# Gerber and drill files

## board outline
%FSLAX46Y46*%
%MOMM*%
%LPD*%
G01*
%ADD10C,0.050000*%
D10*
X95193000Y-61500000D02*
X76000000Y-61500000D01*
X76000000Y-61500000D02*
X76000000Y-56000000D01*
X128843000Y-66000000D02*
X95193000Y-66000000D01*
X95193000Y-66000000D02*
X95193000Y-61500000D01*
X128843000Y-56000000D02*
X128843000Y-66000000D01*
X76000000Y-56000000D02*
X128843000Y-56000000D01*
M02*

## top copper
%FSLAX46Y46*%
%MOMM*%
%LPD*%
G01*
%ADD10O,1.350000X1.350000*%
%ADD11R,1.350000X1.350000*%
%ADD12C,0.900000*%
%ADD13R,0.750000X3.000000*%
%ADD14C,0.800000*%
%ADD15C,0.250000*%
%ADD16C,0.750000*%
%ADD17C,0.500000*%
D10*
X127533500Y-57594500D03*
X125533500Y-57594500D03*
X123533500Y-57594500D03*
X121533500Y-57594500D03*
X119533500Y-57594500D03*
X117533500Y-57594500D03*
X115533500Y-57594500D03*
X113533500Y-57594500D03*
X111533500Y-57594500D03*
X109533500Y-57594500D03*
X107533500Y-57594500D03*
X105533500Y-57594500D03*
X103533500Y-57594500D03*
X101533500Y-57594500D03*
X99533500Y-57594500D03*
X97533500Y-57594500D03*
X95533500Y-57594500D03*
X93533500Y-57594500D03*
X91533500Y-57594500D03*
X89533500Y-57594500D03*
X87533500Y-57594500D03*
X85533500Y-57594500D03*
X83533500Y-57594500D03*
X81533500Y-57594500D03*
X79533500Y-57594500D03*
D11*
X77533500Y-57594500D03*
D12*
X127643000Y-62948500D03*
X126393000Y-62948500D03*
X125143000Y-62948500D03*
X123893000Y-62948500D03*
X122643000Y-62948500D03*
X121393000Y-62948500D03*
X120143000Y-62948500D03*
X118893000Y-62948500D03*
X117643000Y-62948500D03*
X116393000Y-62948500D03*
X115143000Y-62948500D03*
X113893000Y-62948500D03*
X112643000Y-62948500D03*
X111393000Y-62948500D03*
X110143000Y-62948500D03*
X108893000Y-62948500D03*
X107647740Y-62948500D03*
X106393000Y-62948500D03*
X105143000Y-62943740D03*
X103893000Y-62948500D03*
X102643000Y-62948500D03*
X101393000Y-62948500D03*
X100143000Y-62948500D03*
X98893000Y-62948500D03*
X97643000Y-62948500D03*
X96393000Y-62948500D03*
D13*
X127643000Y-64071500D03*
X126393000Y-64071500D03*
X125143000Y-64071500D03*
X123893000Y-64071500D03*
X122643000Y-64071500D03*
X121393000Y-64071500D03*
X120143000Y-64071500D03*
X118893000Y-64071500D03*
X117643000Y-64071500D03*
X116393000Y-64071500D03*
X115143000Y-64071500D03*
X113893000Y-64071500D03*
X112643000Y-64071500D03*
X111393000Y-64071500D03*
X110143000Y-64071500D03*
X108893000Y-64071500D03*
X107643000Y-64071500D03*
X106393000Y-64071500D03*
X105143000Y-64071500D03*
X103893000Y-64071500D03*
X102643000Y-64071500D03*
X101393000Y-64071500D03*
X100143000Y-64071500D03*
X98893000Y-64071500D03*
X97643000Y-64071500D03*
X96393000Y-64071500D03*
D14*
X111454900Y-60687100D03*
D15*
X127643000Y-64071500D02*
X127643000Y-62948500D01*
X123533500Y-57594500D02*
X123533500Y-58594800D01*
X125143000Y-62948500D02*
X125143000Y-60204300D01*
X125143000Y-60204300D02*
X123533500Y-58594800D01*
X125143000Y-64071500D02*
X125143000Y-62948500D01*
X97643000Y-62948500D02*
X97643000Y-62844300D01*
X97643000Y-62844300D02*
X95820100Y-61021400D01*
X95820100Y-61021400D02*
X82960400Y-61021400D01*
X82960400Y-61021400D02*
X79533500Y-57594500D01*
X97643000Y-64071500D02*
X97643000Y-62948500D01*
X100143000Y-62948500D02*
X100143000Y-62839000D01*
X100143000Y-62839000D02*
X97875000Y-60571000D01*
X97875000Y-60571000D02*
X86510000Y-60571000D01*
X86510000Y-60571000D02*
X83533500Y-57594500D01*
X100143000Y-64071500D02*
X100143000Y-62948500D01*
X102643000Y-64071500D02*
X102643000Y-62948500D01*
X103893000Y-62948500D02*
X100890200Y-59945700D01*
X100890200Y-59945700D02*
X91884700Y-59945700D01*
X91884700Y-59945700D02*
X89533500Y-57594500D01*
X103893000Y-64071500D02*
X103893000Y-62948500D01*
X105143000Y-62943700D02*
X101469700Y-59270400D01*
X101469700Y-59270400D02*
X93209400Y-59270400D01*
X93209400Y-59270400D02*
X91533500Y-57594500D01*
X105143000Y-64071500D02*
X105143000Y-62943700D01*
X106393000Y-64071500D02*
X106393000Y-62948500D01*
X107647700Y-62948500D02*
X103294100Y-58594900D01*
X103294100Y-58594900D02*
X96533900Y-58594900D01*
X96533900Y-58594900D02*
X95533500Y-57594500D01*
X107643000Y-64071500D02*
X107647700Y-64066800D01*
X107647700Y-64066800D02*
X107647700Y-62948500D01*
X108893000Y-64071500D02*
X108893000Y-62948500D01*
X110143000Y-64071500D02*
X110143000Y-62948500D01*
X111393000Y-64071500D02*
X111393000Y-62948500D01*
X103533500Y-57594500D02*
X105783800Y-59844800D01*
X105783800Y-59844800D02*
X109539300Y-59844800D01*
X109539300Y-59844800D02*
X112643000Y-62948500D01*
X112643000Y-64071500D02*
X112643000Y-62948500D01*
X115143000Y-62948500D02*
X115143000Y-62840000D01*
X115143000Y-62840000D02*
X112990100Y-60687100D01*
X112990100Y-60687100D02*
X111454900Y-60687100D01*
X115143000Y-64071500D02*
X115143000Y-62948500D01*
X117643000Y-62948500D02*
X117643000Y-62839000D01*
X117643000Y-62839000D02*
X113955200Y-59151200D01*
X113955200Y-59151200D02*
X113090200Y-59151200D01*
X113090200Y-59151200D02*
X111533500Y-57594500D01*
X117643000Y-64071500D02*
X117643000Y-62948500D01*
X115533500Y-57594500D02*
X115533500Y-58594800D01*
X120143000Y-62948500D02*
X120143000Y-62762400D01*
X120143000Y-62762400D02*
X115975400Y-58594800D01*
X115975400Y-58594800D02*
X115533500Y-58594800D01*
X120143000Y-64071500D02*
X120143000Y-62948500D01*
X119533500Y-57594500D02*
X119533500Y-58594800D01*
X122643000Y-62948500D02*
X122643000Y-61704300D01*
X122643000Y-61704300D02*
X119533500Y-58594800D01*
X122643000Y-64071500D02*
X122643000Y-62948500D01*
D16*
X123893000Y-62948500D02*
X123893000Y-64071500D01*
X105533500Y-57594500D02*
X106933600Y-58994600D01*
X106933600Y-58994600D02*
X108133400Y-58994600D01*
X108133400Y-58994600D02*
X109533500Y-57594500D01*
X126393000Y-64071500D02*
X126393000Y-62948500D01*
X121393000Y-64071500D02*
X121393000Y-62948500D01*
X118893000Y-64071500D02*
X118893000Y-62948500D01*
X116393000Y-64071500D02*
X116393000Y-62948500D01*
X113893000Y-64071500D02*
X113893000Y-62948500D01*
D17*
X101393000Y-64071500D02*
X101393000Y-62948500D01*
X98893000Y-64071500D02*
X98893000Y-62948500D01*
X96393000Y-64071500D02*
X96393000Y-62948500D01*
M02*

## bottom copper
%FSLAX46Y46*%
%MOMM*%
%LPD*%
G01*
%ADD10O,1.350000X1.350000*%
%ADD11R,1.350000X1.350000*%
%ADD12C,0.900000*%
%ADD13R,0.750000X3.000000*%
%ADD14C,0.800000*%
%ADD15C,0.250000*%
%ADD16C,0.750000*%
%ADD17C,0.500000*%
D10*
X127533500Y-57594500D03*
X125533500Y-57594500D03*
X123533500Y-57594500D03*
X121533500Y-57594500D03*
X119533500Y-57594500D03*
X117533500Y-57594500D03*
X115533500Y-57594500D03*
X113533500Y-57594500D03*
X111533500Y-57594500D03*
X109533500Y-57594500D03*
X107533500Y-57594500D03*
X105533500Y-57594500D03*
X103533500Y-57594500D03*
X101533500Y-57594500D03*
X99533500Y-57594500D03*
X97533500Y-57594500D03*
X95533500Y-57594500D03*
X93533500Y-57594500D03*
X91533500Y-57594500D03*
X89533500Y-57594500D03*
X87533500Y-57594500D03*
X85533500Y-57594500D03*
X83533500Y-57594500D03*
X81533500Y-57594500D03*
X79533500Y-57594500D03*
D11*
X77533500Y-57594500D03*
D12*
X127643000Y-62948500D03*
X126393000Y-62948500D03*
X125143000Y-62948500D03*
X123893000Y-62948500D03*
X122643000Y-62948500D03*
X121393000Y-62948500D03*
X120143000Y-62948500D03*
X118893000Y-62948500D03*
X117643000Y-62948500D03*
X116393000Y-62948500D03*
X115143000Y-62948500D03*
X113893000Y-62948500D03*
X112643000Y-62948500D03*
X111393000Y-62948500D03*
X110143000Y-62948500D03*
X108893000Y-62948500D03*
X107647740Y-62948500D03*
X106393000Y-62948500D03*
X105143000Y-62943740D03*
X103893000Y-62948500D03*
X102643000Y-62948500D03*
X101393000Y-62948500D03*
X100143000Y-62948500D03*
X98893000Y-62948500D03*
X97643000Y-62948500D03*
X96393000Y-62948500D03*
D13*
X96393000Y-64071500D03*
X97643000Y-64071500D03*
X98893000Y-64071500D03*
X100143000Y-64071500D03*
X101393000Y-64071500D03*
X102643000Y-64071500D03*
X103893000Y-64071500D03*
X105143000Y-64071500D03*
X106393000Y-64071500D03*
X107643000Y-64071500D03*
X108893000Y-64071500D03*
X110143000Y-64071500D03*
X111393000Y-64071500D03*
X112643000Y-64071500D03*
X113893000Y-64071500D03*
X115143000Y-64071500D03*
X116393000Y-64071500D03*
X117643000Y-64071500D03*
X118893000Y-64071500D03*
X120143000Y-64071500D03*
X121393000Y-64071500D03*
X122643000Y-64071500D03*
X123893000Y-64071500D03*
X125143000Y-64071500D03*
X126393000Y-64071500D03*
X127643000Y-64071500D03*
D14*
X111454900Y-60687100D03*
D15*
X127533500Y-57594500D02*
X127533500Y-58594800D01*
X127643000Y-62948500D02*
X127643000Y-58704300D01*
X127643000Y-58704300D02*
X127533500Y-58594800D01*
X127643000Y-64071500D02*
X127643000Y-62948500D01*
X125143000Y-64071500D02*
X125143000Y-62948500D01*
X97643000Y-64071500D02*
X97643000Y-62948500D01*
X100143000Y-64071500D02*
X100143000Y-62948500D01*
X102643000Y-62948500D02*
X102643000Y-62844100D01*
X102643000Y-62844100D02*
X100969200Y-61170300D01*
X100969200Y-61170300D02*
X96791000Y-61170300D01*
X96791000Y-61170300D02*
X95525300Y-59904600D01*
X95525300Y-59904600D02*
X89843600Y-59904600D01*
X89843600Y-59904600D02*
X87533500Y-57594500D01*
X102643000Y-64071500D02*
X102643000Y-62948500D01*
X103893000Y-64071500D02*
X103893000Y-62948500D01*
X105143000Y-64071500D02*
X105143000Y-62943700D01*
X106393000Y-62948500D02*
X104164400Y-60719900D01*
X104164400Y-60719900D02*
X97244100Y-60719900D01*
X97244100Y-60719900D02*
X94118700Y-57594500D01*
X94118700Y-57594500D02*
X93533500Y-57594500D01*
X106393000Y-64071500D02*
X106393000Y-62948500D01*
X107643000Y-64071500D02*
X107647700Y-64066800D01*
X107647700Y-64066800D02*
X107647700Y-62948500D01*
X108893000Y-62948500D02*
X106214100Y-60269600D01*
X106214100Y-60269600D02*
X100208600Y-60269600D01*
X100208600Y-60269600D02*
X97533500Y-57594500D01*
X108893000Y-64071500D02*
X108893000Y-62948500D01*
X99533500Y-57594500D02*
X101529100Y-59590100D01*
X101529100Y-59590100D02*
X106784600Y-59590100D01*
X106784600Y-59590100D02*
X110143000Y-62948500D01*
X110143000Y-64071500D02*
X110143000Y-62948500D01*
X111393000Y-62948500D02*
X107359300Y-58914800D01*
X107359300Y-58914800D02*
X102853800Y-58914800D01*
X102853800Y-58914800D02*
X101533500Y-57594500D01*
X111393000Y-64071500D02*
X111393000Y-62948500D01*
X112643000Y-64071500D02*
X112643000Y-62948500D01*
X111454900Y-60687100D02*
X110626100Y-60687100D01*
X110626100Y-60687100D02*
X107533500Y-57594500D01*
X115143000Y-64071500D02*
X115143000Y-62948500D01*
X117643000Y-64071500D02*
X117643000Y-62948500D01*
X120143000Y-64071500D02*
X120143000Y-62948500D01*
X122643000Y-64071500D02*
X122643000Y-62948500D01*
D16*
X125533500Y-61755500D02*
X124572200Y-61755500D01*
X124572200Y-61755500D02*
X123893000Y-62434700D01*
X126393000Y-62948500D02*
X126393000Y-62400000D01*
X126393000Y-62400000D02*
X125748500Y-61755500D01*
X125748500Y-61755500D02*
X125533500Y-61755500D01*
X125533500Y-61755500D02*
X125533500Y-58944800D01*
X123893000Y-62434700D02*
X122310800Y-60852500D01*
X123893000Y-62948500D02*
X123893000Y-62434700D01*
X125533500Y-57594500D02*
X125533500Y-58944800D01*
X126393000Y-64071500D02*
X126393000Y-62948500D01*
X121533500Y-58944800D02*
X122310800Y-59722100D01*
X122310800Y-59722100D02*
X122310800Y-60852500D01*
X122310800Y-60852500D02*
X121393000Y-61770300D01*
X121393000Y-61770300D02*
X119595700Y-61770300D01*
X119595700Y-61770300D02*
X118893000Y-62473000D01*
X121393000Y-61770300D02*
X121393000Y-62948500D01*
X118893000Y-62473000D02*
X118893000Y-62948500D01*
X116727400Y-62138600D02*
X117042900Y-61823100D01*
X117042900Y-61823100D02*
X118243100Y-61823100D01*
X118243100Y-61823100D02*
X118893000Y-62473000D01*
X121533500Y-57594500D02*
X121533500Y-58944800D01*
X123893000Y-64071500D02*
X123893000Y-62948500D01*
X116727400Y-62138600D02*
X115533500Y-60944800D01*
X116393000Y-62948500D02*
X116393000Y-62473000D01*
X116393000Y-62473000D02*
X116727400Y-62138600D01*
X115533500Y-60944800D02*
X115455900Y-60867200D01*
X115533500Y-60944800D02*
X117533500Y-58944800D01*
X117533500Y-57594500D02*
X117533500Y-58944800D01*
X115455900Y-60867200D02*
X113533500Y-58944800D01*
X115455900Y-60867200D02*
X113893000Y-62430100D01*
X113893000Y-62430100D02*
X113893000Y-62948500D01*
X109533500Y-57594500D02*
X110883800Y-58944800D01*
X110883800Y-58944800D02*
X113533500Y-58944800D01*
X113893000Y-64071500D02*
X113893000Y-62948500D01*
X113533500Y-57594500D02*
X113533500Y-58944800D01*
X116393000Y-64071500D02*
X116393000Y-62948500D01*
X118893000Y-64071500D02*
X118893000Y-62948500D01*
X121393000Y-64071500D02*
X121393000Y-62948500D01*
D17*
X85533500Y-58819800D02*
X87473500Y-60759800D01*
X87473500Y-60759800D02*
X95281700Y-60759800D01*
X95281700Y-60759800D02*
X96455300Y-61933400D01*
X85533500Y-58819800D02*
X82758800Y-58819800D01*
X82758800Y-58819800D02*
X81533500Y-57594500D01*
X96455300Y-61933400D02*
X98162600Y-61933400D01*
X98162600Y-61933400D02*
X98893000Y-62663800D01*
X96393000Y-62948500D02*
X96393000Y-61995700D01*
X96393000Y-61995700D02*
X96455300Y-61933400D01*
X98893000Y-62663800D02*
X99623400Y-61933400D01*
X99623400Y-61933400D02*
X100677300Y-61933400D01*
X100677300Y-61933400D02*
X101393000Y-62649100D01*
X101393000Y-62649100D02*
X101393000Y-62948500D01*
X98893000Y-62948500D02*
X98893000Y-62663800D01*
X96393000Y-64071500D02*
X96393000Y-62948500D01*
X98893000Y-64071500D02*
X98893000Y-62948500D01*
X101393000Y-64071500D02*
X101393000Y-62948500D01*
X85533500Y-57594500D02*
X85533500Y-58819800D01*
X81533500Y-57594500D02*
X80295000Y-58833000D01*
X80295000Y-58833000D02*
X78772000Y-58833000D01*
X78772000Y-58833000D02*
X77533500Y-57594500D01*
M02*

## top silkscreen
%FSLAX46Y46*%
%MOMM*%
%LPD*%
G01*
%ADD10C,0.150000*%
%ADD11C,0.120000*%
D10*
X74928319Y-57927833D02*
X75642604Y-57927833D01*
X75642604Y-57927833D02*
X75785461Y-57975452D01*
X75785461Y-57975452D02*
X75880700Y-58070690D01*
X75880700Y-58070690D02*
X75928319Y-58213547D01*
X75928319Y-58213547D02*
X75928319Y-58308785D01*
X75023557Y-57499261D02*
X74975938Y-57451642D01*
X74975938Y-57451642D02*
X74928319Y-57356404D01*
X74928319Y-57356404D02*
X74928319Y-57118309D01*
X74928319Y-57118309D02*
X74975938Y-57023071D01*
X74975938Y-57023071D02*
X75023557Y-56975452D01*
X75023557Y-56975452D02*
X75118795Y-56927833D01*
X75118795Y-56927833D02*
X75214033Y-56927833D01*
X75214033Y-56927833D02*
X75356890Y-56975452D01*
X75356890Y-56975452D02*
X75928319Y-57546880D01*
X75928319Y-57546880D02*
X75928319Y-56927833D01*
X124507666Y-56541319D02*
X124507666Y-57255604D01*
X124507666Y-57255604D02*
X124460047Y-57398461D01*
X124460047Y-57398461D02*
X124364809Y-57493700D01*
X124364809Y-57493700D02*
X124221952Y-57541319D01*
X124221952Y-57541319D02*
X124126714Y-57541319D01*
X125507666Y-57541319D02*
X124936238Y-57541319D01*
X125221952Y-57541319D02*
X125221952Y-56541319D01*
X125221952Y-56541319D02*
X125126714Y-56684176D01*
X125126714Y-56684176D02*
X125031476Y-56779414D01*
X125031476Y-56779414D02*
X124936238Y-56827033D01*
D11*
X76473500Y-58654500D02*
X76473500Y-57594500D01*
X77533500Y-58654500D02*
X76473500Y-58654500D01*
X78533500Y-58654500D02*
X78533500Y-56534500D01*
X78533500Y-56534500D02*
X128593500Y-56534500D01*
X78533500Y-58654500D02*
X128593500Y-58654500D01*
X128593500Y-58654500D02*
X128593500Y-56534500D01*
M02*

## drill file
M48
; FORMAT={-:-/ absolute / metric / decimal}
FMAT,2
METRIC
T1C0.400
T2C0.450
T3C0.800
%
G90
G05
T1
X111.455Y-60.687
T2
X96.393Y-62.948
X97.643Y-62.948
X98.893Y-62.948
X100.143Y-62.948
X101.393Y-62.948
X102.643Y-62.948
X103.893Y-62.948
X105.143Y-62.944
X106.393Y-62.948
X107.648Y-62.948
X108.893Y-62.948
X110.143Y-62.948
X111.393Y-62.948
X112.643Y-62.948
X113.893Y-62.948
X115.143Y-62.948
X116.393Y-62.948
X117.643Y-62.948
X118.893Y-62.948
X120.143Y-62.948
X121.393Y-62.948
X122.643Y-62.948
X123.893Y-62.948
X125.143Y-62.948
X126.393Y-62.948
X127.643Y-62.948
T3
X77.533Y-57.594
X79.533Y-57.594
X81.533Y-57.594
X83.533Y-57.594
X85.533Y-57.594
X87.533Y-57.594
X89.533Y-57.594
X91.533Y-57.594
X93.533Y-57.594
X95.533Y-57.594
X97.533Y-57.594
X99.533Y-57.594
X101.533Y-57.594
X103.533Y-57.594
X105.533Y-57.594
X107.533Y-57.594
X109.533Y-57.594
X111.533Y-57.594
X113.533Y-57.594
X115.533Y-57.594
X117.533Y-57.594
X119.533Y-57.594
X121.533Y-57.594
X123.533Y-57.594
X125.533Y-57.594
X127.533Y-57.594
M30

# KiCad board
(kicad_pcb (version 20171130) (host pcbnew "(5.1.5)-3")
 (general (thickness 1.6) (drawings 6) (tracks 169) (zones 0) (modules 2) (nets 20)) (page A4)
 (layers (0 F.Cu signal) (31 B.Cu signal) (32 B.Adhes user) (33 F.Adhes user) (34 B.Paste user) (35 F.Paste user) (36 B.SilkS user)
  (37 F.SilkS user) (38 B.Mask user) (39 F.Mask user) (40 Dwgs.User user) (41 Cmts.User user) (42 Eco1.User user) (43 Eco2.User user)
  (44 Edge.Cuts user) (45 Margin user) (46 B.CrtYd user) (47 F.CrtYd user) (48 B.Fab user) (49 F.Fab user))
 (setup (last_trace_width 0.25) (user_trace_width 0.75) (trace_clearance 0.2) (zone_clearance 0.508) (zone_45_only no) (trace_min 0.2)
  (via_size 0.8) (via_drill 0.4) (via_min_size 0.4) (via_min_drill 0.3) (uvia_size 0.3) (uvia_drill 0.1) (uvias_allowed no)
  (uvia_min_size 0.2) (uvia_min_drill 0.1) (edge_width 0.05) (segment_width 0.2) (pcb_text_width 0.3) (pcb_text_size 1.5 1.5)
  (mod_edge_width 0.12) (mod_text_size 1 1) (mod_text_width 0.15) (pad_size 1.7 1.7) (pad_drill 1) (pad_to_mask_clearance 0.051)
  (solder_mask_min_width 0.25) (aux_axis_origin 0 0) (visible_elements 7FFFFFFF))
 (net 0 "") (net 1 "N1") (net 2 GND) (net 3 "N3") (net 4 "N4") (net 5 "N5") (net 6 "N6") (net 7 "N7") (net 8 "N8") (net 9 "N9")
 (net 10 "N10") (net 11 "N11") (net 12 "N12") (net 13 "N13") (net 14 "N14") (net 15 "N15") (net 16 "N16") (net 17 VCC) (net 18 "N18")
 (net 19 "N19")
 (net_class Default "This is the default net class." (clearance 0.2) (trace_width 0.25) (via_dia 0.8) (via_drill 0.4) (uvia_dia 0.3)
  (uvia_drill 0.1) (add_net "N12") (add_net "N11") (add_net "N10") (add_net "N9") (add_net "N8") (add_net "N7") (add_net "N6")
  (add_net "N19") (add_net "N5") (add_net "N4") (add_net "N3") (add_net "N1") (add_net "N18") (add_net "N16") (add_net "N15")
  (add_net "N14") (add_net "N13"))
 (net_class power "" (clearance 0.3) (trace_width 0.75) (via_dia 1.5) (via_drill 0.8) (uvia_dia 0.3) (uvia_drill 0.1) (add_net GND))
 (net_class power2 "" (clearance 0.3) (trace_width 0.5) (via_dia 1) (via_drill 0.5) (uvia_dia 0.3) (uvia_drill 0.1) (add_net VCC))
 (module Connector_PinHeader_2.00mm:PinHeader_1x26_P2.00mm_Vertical (layer F.Cu) (at 77.5335 57.5945 90)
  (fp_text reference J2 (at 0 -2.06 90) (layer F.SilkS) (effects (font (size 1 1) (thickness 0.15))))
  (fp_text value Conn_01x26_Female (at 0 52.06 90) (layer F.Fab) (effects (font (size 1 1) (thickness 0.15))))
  (fp_line (start -1.06 -1.06) (end 0 -1.06) (layer F.SilkS) (width 0.12))
  (fp_line (start -1.06 0) (end -1.06 -1.06) (layer F.SilkS) (width 0.12))
  (fp_line (start -1.06 1) (end 1.06 1) (layer F.SilkS) (width 0.12))
  (fp_line (start 1.06 1) (end 1.06 51.06) (layer F.SilkS) (width 0.12))
  (fp_line (start -1.06 1) (end -1.06 51.06) (layer F.SilkS) (width 0.12))
  (fp_line (start -1.06 51.06) (end 1.06 51.06) (layer F.SilkS) (width 0.12))
  (pad 26 thru_hole oval (at 0 50 90) (size 1.35 1.35) (drill 0.8) (layers *.Cu *.Mask) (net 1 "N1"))
  (pad 25 thru_hole oval (at 0 48 90) (size 1.35 1.35) (drill 0.8) (layers *.Cu *.Mask) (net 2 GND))
  (pad 24 thru_hole oval (at 0 46 90) (size 1.35 1.35) (drill 0.8) (layers *.Cu *.Mask) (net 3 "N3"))
  (pad 23 thru_hole oval (at 0 44 90) (size 1.35 1.35) (drill 0.8) (layers *.Cu *.Mask) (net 2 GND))
  (pad 22 thru_hole oval (at 0 42 90) (size 1.35 1.35) (drill 0.8) (layers *.Cu *.Mask) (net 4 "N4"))
  (pad 21 thru_hole oval (at 0 40 90) (size 1.35 1.35) (drill 0.8) (layers *.Cu *.Mask) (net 2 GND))
  (pad 20 thru_hole oval (at 0 38 90) (size 1.35 1.35) (drill 0.8) (layers *.Cu *.Mask) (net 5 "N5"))
  (pad 19 thru_hole oval (at 0 36 90) (size 1.35 1.35) (drill 0.8) (layers *.Cu *.Mask) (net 2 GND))
  (pad 18 thru_hole oval (at 0 34 90) (size 1.35 1.35) (drill 0.8) (layers *.Cu *.Mask) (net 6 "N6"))
  (pad 17 thru_hole oval (at 0 32 90) (size 1.35 1.35) (drill 0.8) (layers *.Cu *.Mask) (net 2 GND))
  (pad 16 thru_hole oval (at 0 30 90) (size 1.35 1.35) (drill 0.8) (layers *.Cu *.Mask) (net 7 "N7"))
  (pad 15 thru_hole oval (at 0 28 90) (size 1.35 1.35) (drill 0.8) (layers *.Cu *.Mask) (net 2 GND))
  (pad 14 thru_hole oval (at 0 26 90) (size 1.35 1.35) (drill 0.8) (layers *.Cu *.Mask) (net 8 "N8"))
  (pad 13 thru_hole oval (at 0 24 90) (size 1.35 1.35) (drill 0.8) (layers *.Cu *.Mask) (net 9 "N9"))
  (pad 12 thru_hole oval (at 0 22 90) (size 1.35 1.35) (drill 0.8) (layers *.Cu *.Mask) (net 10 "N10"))
  (pad 11 thru_hole oval (at 0 20 90) (size 1.35 1.35) (drill 0.8) (layers *.Cu *.Mask) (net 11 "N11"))
  (pad 10 thru_hole oval (at 0 18 90) (size 1.35 1.35) (drill 0.8) (layers *.Cu *.Mask) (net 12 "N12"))
  (pad 9 thru_hole oval (at 0 16 90) (size 1.35 1.35) (drill 0.8) (layers *.Cu *.Mask) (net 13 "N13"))
  (pad 8 thru_hole oval (at 0 14 90) (size 1.35 1.35) (drill 0.8) (layers *.Cu *.Mask) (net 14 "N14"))
  (pad 7 thru_hole oval (at 0 12 90) (size 1.35 1.35) (drill 0.8) (layers *.Cu *.Mask) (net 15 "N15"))
  (pad 6 thru_hole oval (at 0 10 90) (size 1.35 1.35) (drill 0.8) (layers *.Cu *.Mask) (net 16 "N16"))
  (pad 5 thru_hole oval (at 0 8 90) (size 1.35 1.35) (drill 0.8) (layers *.Cu *.Mask) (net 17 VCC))
  (pad 4 thru_hole oval (at 0 6 90) (size 1.35 1.35) (drill 0.8) (layers *.Cu *.Mask) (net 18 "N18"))
  (pad 3 thru_hole oval (at 0 4 90) (size 1.35 1.35) (drill 0.8) (layers *.Cu *.Mask) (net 17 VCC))
  (pad 2 thru_hole oval (at 0 2 90) (size 1.35 1.35) (drill 0.8) (layers *.Cu *.Mask) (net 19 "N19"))
  (pad 1 thru_hole rect (at 0 0 90) (size 1.35 1.35) (drill 0.8) (layers *.Cu *.Mask) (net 17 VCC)))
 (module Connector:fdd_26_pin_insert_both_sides (layer F.Cu) (at 96.393 64.1985)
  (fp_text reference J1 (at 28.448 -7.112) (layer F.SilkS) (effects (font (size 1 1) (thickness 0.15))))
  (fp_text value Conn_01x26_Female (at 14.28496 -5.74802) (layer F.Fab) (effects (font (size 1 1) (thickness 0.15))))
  (pad 26 thru_hole circle (at 31.25 -1.25) (size 0.9 0.9) (drill 0.45) (layers *.Cu *.Mask) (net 1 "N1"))
  (pad 25 thru_hole circle (at 30 -1.25) (size 0.9 0.9) (drill 0.45) (layers *.Cu *.Mask) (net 2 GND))
  (pad 24 thru_hole circle (at 28.75 -1.25) (size 0.9 0.9) (drill 0.45) (layers *.Cu *.Mask) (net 3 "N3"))
  (pad 23 thru_hole circle (at 27.5 -1.25) (size 0.9 0.9) (drill 0.45) (layers *.Cu *.Mask) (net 2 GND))
  (pad 22 thru_hole circle (at 26.25 -1.25) (size 0.9 0.9) (drill 0.45) (layers *.Cu *.Mask) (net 4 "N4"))
  (pad 21 thru_hole circle (at 25 -1.25) (size 0.9 0.9) (drill 0.45) (layers *.Cu *.Mask) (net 2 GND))
  (pad 20 thru_hole circle (at 23.75 -1.25) (size 0.9 0.9) (drill 0.45) (layers *.Cu *.Mask) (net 5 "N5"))
  (pad 19 thru_hole circle (at 22.5 -1.25) (size 0.9 0.9) (drill 0.45) (layers *.Cu *.Mask) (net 2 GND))
  (pad 18 thru_hole circle (at 21.25 -1.25) (size 0.9 0.9) (drill 0.45) (layers *.Cu *.Mask) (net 6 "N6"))
  (pad 17 thru_hole circle (at 20 -1.25) (size 0.9 0.9) (drill 0.45) (layers *.Cu *.Mask) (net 2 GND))
  (pad 16 thru_hole circle (at 18.75 -1.25) (size 0.9 0.9) (drill 0.45) (layers *.Cu *.Mask) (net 7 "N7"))
  (pad 15 thru_hole circle (at 17.5 -1.25 90) (size 0.9 0.9) (drill 0.45) (layers *.Cu *.Mask) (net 2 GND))
  (pad 14 thru_hole circle (at 16.25 -1.25) (size 0.9 0.9) (drill 0.45) (layers *.Cu *.Mask) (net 8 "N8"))
  (pad 13 thru_hole circle (at 15 -1.25) (size 0.9 0.9) (drill 0.45) (layers *.Cu *.Mask) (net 9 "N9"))
  (pad 12 thru_hole circle (at 13.75 -1.25) (size 0.9 0.9) (drill 0.45) (layers *.Cu *.Mask) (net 10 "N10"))
  (pad 11 thru_hole circle (at 12.5 -1.25) (size 0.9 0.9) (drill 0.45) (layers *.Cu *.Mask) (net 11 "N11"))
  (pad 10 thru_hole circle (at 11.25474 -1.25) (size 0.9 0.9) (drill 0.45) (layers *.Cu *.Mask) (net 12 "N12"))
  (pad 9 thru_hole circle (at 10 -1.25) (size 0.9 0.9) (drill 0.45) (layers *.Cu *.Mask) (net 13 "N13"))
  (pad 8 thru_hole circle (at 8.75 -1.25476) (size 0.9 0.9) (drill 0.45) (layers *.Cu *.Mask) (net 14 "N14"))
  (pad 7 thru_hole circle (at 7.5 -1.25) (size 0.9 0.9) (drill 0.45) (layers *.Cu *.Mask) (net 15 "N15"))
  (pad 6 thru_hole circle (at 6.25 -1.25) (size 0.9 0.9) (drill 0.45) (layers *.Cu *.Mask) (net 16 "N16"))
  (pad 5 thru_hole circle (at 5 -1.25) (size 0.9 0.9) (drill 0.45) (layers *.Cu *.Mask) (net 17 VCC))
  (pad 4 thru_hole circle (at 3.75 -1.25) (size 0.9 0.9) (drill 0.45) (layers *.Cu *.Mask) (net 18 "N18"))
  (pad 3 thru_hole circle (at 2.5 -1.25) (size 0.9 0.9) (drill 0.45) (layers *.Cu *.Mask) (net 17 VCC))
  (pad 2 thru_hole circle (at 1.25 -1.25 90) (size 0.9 0.9) (drill 0.45) (layers *.Cu *.Mask) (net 19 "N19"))
  (pad 1 thru_hole circle (at 0 -1.25) (size 0.9 0.9) (drill 0.45) (layers *.Cu *.Mask) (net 17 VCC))
  (pad 26 connect rect (at 31.25 -0.127) (size 0.75 3) (layers F.Cu F.Mask) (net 1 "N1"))
  (pad 25 connect rect (at 30 -0.127) (size 0.75 3) (layers F.Cu F.Mask) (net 2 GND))
  (pad 24 connect rect (at 28.75 -0.127) (size 0.75 3) (layers F.Cu F.Mask) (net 3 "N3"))
  (pad 23 connect rect (at 27.5 -0.127) (size 0.75 3) (layers F.Cu F.Mask) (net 2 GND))
  (pad 22 connect rect (at 26.25 -0.127) (size 0.75 3) (layers F.Cu F.Mask) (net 4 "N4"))
  (pad 21 connect rect (at 25 -0.127) (size 0.75 3) (layers F.Cu F.Mask) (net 2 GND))
  (pad 20 connect rect (at 23.75 -0.127) (size 0.75 3) (layers F.Cu F.Mask) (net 5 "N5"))
  (pad 19 connect rect (at 22.5 -0.127) (size 0.75 3) (layers F.Cu F.Mask) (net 2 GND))
  (pad 18 connect rect (at 21.25 -0.127) (size 0.75 3) (layers F.Cu F.Mask) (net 6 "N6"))
  (pad 17 connect rect (at 20 -0.127) (size 0.75 3) (layers F.Cu F.Mask) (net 2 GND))
  (pad 16 connect rect (at 18.75 -0.127) (size 0.75 3) (layers F.Cu F.Mask) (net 7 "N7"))
  (pad 15 connect rect (at 17.5 -0.127) (size 0.75 3) (layers F.Cu F.Mask) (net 2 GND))
  (pad 14 connect rect (at 16.25 -0.127) (size 0.75 3) (layers F.Cu F.Mask) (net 8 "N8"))
  (pad 13 connect rect (at 15 -0.127) (size 0.75 3) (layers F.Cu F.Mask) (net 9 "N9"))
  (pad 12 connect rect (at 13.75 -0.127) (size 0.75 3) (layers F.Cu F.Mask) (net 10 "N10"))
  (pad 11 connect rect (at 12.5 -0.127) (size 0.75 3) (layers F.Cu F.Mask) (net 11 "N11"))
  (pad 10 connect rect (at 11.25 -0.127) (size 0.75 3) (layers F.Cu F.Mask) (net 12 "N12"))
  (pad 9 connect rect (at 10 -0.127) (size 0.75 3) (layers F.Cu F.Mask) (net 13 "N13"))
  (pad 8 connect rect (at 8.75 -0.127) (size 0.75 3) (layers F.Cu F.Mask) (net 14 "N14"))
  (pad 7 connect rect (at 7.5 -0.127) (size 0.75 3) (layers F.Cu F.Mask) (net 15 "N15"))
  (pad 6 connect rect (at 6.25 -0.127) (size 0.75 3) (layers F.Cu F.Mask) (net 16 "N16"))
  (pad 5 connect rect (at 5 -0.127) (size 0.75 3) (layers F.Cu F.Mask) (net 17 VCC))
  (pad 4 connect rect (at 3.75 -0.127) (size 0.75 3) (layers F.Cu F.Mask) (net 18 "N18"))
  (pad 3 connect rect (at 2.5 -0.127) (size 0.75 3) (layers F.Cu F.Mask) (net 17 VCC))
  (pad 2 connect rect (at 1.25 -0.127) (size 0.75 3) (layers F.Cu F.Mask) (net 19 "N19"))
  (pad 1 connect rect (at 0 -0.127) (size 0.75 3) (layers F.Cu F.Mask) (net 17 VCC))
  (pad 1 connect rect (at 0 -0.127) (size 0.75 3) (layers B.Cu B.Mask) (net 17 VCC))
  (pad 2 connect rect (at 1.25 -0.127) (size 0.75 3) (layers B.Cu B.Mask) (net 19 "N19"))
  (pad 3 connect rect (at 2.5 -0.127) (size 0.75 3) (layers B.Cu B.Mask) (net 17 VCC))
  (pad 4 connect rect (at 3.75 -0.127) (size 0.75 3) (layers B.Cu B.Mask) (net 18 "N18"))
  (pad 5 connect rect (at 5 -0.127) (size 0.75 3) (layers B.Cu B.Mask) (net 17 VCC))
  (pad 6 connect rect (at 6.25 -0.127) (size 0.75 3) (layers B.Cu B.Mask) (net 16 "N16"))
  (pad 7 connect rect (at 7.5 -0.127) (size 0.75 3) (layers B.Cu B.Mask) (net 15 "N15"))
  (pad 8 connect rect (at 8.75 -0.127) (size 0.75 3) (layers B.Cu B.Mask) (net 14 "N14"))
  (pad 9 connect rect (at 10 -0.127) (size 0.75 3) (layers B.Cu B.Mask) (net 13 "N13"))
  (pad 10 connect rect (at 11.25 -0.127) (size 0.75 3) (layers B.Cu B.Mask) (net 12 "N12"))
  (pad 11 connect rect (at 12.5 -0.127) (size 0.75 3) (layers B.Cu B.Mask) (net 11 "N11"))
  (pad 12 connect rect (at 13.75 -0.127) (size 0.75 3) (layers B.Cu B.Mask) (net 10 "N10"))
  (pad 13 connect rect (at 15 -0.127) (size 0.75 3) (layers B.Cu B.Mask) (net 9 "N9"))
  (pad 14 connect rect (at 16.25 -0.127) (size 0.75 3) (layers B.Cu B.Mask) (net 8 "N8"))
  (pad 15 connect rect (at 17.5 -0.127) (size 0.75 3) (layers B.Cu B.Mask) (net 2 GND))
  (pad 16 connect rect (at 18.75 -0.127) (size 0.75 3) (layers B.Cu B.Mask) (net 7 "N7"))
  (pad 17 connect rect (at 20 -0.127) (size 0.75 3) (layers B.Cu B.Mask) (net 2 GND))
  (pad 18 connect rect (at 21.25 -0.127) (size 0.75 3) (layers B.Cu B.Mask) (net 6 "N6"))
  (pad 19 connect rect (at 22.5 -0.127) (size 0.75 3) (layers B.Cu B.Mask) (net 2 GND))
  (pad 20 connect rect (at 23.75 -0.127) (size 0.75 3) (layers B.Cu B.Mask) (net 5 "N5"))
  (pad 21 connect rect (at 25 -0.127) (size 0.75 3) (layers B.Cu B.Mask) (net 2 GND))
  (pad 22 connect rect (at 26.25 -0.127) (size 0.75 3) (layers B.Cu B.Mask) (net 4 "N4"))
  (pad 23 connect rect (at 27.5 -0.127) (size 0.75 3) (layers B.Cu B.Mask) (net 2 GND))
  (pad 24 connect rect (at 28.75 -0.127) (size 0.75 3) (layers B.Cu B.Mask) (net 3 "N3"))
  (pad 25 connect rect (at 30 -0.127) (size 0.75 3) (layers B.Cu B.Mask) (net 2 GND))
  (pad 26 connect rect (at 31.25 -0.127) (size 0.75 3) (layers B.Cu B.Mask) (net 1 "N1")))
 (gr_line (start 95.193 61.5) (end 76 61.5) (layer Edge.Cuts) (width 0.05))
 (gr_line (start 76 61.5) (end 76 56) (layer Edge.Cuts) (width 0.05))
 (gr_line (start 128.843 66) (end 95.193 66) (layer Edge.Cuts) (width 0.05))
 (gr_line (start 95.193 66) (end 95.193 61.5) (layer Edge.Cuts) (width 0.05))
 (gr_line (start 128.843 56) (end 128.843 66) (layer Edge.Cuts) (width 0.05))
 (gr_line (start 76 56) (end 128.843 56) (layer Edge.Cuts) (width 0.05))
 (segment (start 127.5335 57.5945) (end 127.5335 58.5948) (width 0.25) (layer B.Cu) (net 1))
 (segment (start 127.643 62.9485) (end 127.643 58.7043) (width 0.25) (layer B.Cu) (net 1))
 (segment (start 127.643 58.7043) (end 127.5335 58.5948) (width 0.25) (layer B.Cu) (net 1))
 (segment (start 127.643 64.0715) (end 127.643 62.9485) (width 0.25) (layer B.Cu) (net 1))
 (segment (start 127.643 64.0715) (end 127.643 62.9485) (width 0.25) (layer F.Cu) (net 1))
 (segment (start 123.5335 57.5945) (end 123.5335 58.5948) (width 0.25) (layer F.Cu) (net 3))
 (segment (start 125.143 62.9485) (end 125.143 60.2043) (width 0.25) (layer F.Cu) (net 3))
 (segment (start 125.143 60.2043) (end 123.5335 58.5948) (width 0.25) (layer F.Cu) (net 3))
 (segment (start 125.143 64.0715) (end 125.143 62.9485) (width 0.25) (layer F.Cu) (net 3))
 (segment (start 125.143 64.0715) (end 125.143 62.9485) (width 0.25) (layer B.Cu) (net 3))
 (segment (start 97.643 62.9485) (end 97.643 62.8443) (width 0.25) (layer F.Cu) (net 19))
 (segment (start 97.643 62.8443) (end 95.8201 61.0214) (width 0.25) (layer F.Cu) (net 19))
 (segment (start 95.8201 61.0214) (end 82.9604 61.0214) (width 0.25) (layer F.Cu) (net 19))
 (segment (start 82.9604 61.0214) (end 79.5335 57.5945) (width 0.25) (layer F.Cu) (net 19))
 (segment (start 97.643 64.0715) (end 97.643 62.9485) (width 0.25) (layer F.Cu) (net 19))
 (segment (start 97.643 64.0715) (end 97.643 62.9485) (width 0.25) (layer B.Cu) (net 19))
 (segment (start 100.143 62.9485) (end 100.143 62.839) (width 0.25) (layer F.Cu) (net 18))
 (segment (start 100.143 62.839) (end 97.875 60.571) (width 0.25) (layer F.Cu) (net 18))
 (segment (start 97.875 60.571) (end 86.51 60.571) (width 0.25) (layer F.Cu) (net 18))
 (segment (start 86.51 60.571) (end 83.5335 57.5945) (width 0.25) (layer F.Cu) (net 18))
 (segment (start 100.143 64.0715) (end 100.143 62.9485) (width 0.25) (layer F.Cu) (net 18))
 (segment (start 100.143 64.0715) (end 100.143 62.9485) (width 0.25) (layer B.Cu) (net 18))
 (segment (start 102.643 62.9485) (end 102.643 62.8441) (width 0.25) (layer B.Cu) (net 16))
 (segment (start 102.643 62.8441) (end 100.9692 61.1703) (width 0.25) (layer B.Cu) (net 16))
 (segment (start 100.9692 61.1703) (end 96.791 61.1703) (width 0.25) (layer B.Cu) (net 16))
 (segment (start 96.791 61.1703) (end 95.5253 59.9046) (width 0.25) (layer B.Cu) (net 16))
 (segment (start 95.5253 59.9046) (end 89.8436 59.9046) (width 0.25) (layer B.Cu) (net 16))
 (segment (start 89.8436 59.9046) (end 87.5335 57.5945) (width 0.25) (layer B.Cu) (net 16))
 (segment (start 102.643 64.0715) (end 102.643 62.9485) (width 0.25) (layer B.Cu) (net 16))
 (segment (start 102.643 64.0715) (end 102.643 62.9485) (width 0.25) (layer F.Cu) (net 16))
 (segment (start 103.893 62.9485) (end 100.8902 59.9457) (width 0.25) (layer F.Cu) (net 15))
 (segment (start 100.8902 59.9457) (end 91.8847 59.9457) (width 0.25) (layer F.Cu) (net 15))
 (segment (start 91.8847 59.9457) (end 89.5335 57.5945) (width 0.25) (layer F.Cu) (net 15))
 (segment (start 103.893 64.0715) (end 103.893 62.9485) (width 0.25) (layer F.Cu) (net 15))
 (segment (start 103.893 64.0715) (end 103.893 62.9485) (width 0.25) (layer B.Cu) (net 15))
 (segment (start 105.143 62.9437) (end 101.4697 59.2704) (width 0.25) (layer F.Cu) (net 14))
 (segment (start 101.4697 59.2704) (end 93.2094 59.2704) (width 0.25) (layer F.Cu) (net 14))
 (segment (start 93.2094 59.2704) (end 91.5335 57.5945) (width 0.25) (layer F.Cu) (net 14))
 (segment (start 105.143 64.0715) (end 105.143 62.9437) (width 0.25) (layer F.Cu) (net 14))
 (segment (start 105.143 64.0715) (end 105.143 62.9437) (width 0.25) (layer B.Cu) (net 14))
 (segment (start 106.393 62.9485) (end 104.1644 60.7199) (width 0.25) (layer B.Cu) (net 13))
 (segment (start 104.1644 60.7199) (end 97.2441 60.7199) (width 0.25) (layer B.Cu) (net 13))
 (segment (start 97.2441 60.7199) (end 94.1187 57.5945) (width 0.25) (layer B.Cu) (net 13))
 (segment (start 94.1187 57.5945) (end 93.5335 57.5945) (width 0.25) (layer B.Cu) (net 13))
 (segment (start 106.393 64.0715) (end 106.393 62.9485) (width 0.25) (layer B.Cu) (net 13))
 (segment (start 106.393 64.0715) (end 106.393 62.9485) (width 0.25) (layer F.Cu) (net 13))
 (segment (start 107.6477 62.9485) (end 103.2941 58.5949) (width 0.25) (layer F.Cu) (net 12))
 (segment (start 103.2941 58.5949) (end 96.5339 58.5949) (width 0.25) (layer F.Cu) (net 12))
 (segment (start 96.5339 58.5949) (end 95.5335 57.5945) (width 0.25) (layer F.Cu) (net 12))
 (segment (start 107.643 64.0715) (end 107.6477 64.0668) (width 0.25) (layer F.Cu) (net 12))
 (segment (start 107.6477 64.0668) (end 107.6477 62.9485) (width 0.25) (layer F.Cu) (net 12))
 (segment (start 107.643 64.0715) (end 107.6477 64.0668) (width 0.25) (layer B.Cu) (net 12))
 (segment (start 107.6477 64.0668) (end 107.6477 62.9485) (width 0.25) (layer B.Cu) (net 12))
 (segment (start 108.893 62.9485) (end 106.2141 60.2696) (width 0.25) (layer B.Cu) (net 11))
 (segment (start 106.2141 60.2696) (end 100.2086 60.2696) (width 0.25) (layer B.Cu) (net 11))
 (segment (start 100.2086 60.2696) (end 97.5335 57.5945) (width 0.25) (layer B.Cu) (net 11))
 (segment (start 108.893 64.0715) (end 108.893 62.9485) (width 0.25) (layer B.Cu) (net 11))
 (segment (start 108.893 64.0715) (end 108.893 62.9485) (width 0.25) (layer F.Cu) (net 11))
 (segment (start 99.5335 57.5945) (end 101.5291 59.5901) (width 0.25) (layer B.Cu) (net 10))
 (segment (start 101.5291 59.5901) (end 106.7846 59.5901) (width 0.25) (layer B.Cu) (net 10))
 (segment (start 106.7846 59.5901) (end 110.143 62.9485) (width 0.25) (layer B.Cu) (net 10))
 (segment (start 110.143 64.0715) (end 110.143 62.9485) (width 0.25) (layer B.Cu) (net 10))
 (segment (start 110.143 64.0715) (end 110.143 62.9485) (width 0.25) (layer F.Cu) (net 10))
 (segment (start 111.393 62.9485) (end 107.3593 58.9148) (width 0.25) (layer B.Cu) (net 9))
 (segment (start 107.3593 58.9148) (end 102.8538 58.9148) (width 0.25) (layer B.Cu) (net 9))
 (segment (start 102.8538 58.9148) (end 101.5335 57.5945) (width 0.25) (layer B.Cu) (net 9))
 (segment (start 111.393 64.0715) (end 111.393 62.9485) (width 0.25) (layer B.Cu) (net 9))
 (segment (start 111.393 64.0715) (end 111.393 62.9485) (width 0.25) (layer F.Cu) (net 9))
 (segment (start 103.5335 57.5945) (end 105.7838 59.8448) (width 0.25) (layer F.Cu) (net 8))
 (segment (start 105.7838 59.8448) (end 109.5393 59.8448) (width 0.25) (layer F.Cu) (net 8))
 (segment (start 109.5393 59.8448) (end 112.643 62.9485) (width 0.25) (layer F.Cu) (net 8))
 (segment (start 112.643 64.0715) (end 112.643 62.9485) (width 0.25) (layer F.Cu) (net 8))
 (segment (start 112.643 64.0715) (end 112.643 62.9485) (width 0.25) (layer B.Cu) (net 8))
 (segment (start 115.143 62.9485) (end 115.143 62.84) (width 0.25) (layer F.Cu) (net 7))
 (segment (start 115.143 62.84) (end 112.9901 60.6871) (width 0.25) (layer F.Cu) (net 7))
 (segment (start 112.9901 60.6871) (end 111.4549 60.6871) (width 0.25) (layer F.Cu) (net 7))
 (segment (start 111.4549 60.6871) (end 110.6261 60.6871) (width 0.25) (layer B.Cu) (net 7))
 (segment (start 110.6261 60.6871) (end 107.5335 57.5945) (width 0.25) (layer B.Cu) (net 7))
 (segment (start 115.143 64.0715) (end 115.143 62.9485) (width 0.25) (layer F.Cu) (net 7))
 (segment (start 115.143 64.0715) (end 115.143 62.9485) (width 0.25) (layer B.Cu) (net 7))
 (via (at 111.4549 60.6871) (size 0.8) (layers F.Cu B.Cu) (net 7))
 (segment (start 117.643 62.9485) (end 117.643 62.839) (width 0.25) (layer F.Cu) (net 6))
 (segment (start 117.643 62.839) (end 113.9552 59.1512) (width 0.25) (layer F.Cu) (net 6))
 (segment (start 113.9552 59.1512) (end 113.0902 59.1512) (width 0.25) (layer F.Cu) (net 6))
 (segment (start 113.0902 59.1512) (end 111.5335 57.5945) (width 0.25) (layer F.Cu) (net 6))
 (segment (start 117.643 64.0715) (end 117.643 62.9485) (width 0.25) (layer F.Cu) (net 6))
 (segment (start 117.643 64.0715) (end 117.643 62.9485) (width 0.25) (layer B.Cu) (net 6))
 (segment (start 115.5335 57.5945) (end 115.5335 58.5948) (width 0.25) (layer F.Cu) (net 5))
 (segment (start 120.143 62.9485) (end 120.143 62.7624) (width 0.25) (layer F.Cu) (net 5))
 (segment (start 120.143 62.7624) (end 115.9754 58.5948) (width 0.25) (layer F.Cu) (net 5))
 (segment (start 115.9754 58.5948) (end 115.5335 58.5948) (width 0.25) (layer F.Cu) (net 5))
 (segment (start 120.143 64.0715) (end 120.143 62.9485) (width 0.25) (layer F.Cu) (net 5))
 (segment (start 120.143 64.0715) (end 120.143 62.9485) (width 0.25) (layer B.Cu) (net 5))
 (segment (start 119.5335 57.5945) (end 119.5335 58.5948) (width 0.25) (layer F.Cu) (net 4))
 (segment (start 122.643 62.9485) (end 122.643 61.7043) (width 0.25) (layer F.Cu) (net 4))
 (segment (start 122.643 61.7043) (end 119.5335 58.5948) (width 0.25) (layer F.Cu) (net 4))
 (segment (start 122.643 64.0715) (end 122.643 62.9485) (width 0.25) (layer F.Cu) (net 4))
 (segment (start 122.643 64.0715) (end 122.643 62.9485) (width 0.25) (layer B.Cu) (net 4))
 (segment (start 125.5335 61.7555) (end 124.5722 61.7555) (width 0.75) (layer B.Cu) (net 2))
 (segment (start 124.5722 61.7555) (end 123.893 62.4347) (width 0.75) (layer B.Cu) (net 2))
 (segment (start 126.393 62.9485) (end 126.393 62.4) (width 0.75) (layer B.Cu) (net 2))
 (segment (start 126.393 62.4) (end 125.7485 61.7555) (width 0.75) (layer B.Cu) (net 2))
 (segment (start 125.7485 61.7555) (end 125.5335 61.7555) (width 0.75) (layer B.Cu) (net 2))
 (segment (start 125.5335 61.7555) (end 125.5335 58.9448) (width 0.75) (layer B.Cu) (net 2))
 (segment (start 123.893 62.4347) (end 122.3108 60.8525) (width 0.75) (layer B.Cu) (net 2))
 (segment (start 123.893 62.9485) (end 123.893 62.4347) (width 0.75) (layer B.Cu) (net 2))
 (segment (start 125.5335 57.5945) (end 125.5335 58.9448) (width 0.75) (layer B.Cu) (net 2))
 (segment (start 126.393 64.0715) (end 126.393 62.9485) (width 0.75) (layer B.Cu) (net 2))
 (segment (start 123.893 62.9485) (end 123.893 64.0715) (width 0.75) (layer F.Cu) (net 2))
 (segment (start 121.5335 58.9448) (end 122.3108 59.7221) (width 0.75) (layer B.Cu) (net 2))
 (segment (start 122.3108 59.7221) (end 122.3108 60.8525) (width 0.75) (layer B.Cu) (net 2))
 (segment (start 122.3108 60.8525) (end 121.393 61.7703) (width 0.75) (layer B.Cu) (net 2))
 (segment (start 121.393 61.7703) (end 119.5957 61.7703) (width 0.75) (layer B.Cu) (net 2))
 (segment (start 119.5957 61.7703) (end 118.893 62.473) (width 0.75) (layer B.Cu) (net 2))
 (segment (start 121.393 61.7703) (end 121.393 62.9485) (width 0.75) (layer B.Cu) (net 2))
 (segment (start 118.893 62.473) (end 118.893 62.9485) (width 0.75) (layer B.Cu) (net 2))
 (segment (start 116.7274 62.1386) (end 117.0429 61.8231) (width 0.75) (layer B.Cu) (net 2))
 (segment (start 117.0429 61.8231) (end 118.2431 61.8231) (width 0.75) (layer B.Cu) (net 2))
 (segment (start 118.2431 61.8231) (end 118.893 62.473) (width 0.75) (layer B.Cu) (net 2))
 (segment (start 121.5335 57.5945) (end 121.5335 58.9448) (width 0.75) (layer B.Cu) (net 2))
 (segment (start 123.893 64.0715) (end 123.893 62.9485) (width 0.75) (layer B.Cu) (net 2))
 (segment (start 116.7274 62.1386) (end 115.5335 60.9448) (width 0.75) (layer B.Cu) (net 2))
 (segment (start 116.393 62.9485) (end 116.393 62.473) (width 0.75) (layer B.Cu) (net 2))
 (segment (start 116.393 62.473) (end 116.7274 62.1386) (width 0.75) (layer B.Cu) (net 2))
 (segment (start 115.5335 60.9448) (end 115.4559 60.8672) (width 0.75) (layer B.Cu) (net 2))
 (segment (start 115.5335 60.9448) (end 117.5335 58.9448) (width 0.75) (layer B.Cu) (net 2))
 (segment (start 117.5335 57.5945) (end 117.5335 58.9448) (width 0.75) (layer B.Cu) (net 2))
 (segment (start 115.4559 60.8672) (end 113.5335 58.9448) (width 0.75) (layer B.Cu) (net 2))
 (segment (start 115.4559 60.8672) (end 113.893 62.4301) (width 0.75) (layer B.Cu) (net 2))
 (segment (start 113.893 62.4301) (end 113.893 62.9485) (width 0.75) (layer B.Cu) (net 2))
 (segment (start 109.5335 57.5945) (end 110.8838 58.9448) (width 0.75) (layer B.Cu) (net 2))
 (segment (start 110.8838 58.9448) (end 113.5335 58.9448) (width 0.75) (layer B.Cu) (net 2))
 (segment (start 113.893 64.0715) (end 113.893 62.9485) (width 0.75) (layer B.Cu) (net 2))
 (segment (start 113.5335 57.5945) (end 113.5335 58.9448) (width 0.75) (layer B.Cu) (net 2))
 (segment (start 105.5335 57.5945) (end 106.9336 58.9946) (width 0.75) (layer F.Cu) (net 2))
 (segment (start 106.9336 58.9946) (end 108.1334 58.9946) (width 0.75) (layer F.Cu) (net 2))
 (segment (start 108.1334 58.9946) (end 109.5335 57.5945) (width 0.75) (layer F.Cu) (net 2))
 (segment (start 126.393 64.0715) (end 126.393 62.9485) (width 0.75) (layer F.Cu) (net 2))
 (segment (start 121.393 64.0715) (end 121.393 62.9485) (width 0.75) (layer F.Cu) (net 2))
 (segment (start 118.893 64.0715) (end 118.893 62.9485) (width 0.75) (layer F.Cu) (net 2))
 (segment (start 116.393 64.0715) (end 116.393 62.9485) (width 0.75) (layer F.Cu) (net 2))
 (segment (start 113.893 64.0715) (end 113.893 62.9485) (width 0.75) (layer F.Cu) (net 2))
 (segment (start 116.393 64.0715) (end 116.393 62.9485) (width 0.75) (layer B.Cu) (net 2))
 (segment (start 118.893 64.0715) (end 118.893 62.9485) (width 0.75) (layer B.Cu) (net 2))
 (segment (start 121.393 64.0715) (end 121.393 62.9485) (width 0.75) (layer B.Cu) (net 2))
 (segment (start 85.5335 58.8198) (end 87.4735 60.7598) (width 0.5) (layer B.Cu) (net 17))
 (segment (start 87.4735 60.7598) (end 95.2817 60.7598) (width 0.5) (layer B.Cu) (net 17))
 (segment (start 95.2817 60.7598) (end 96.4553 61.9334) (width 0.5) (layer B.Cu) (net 17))
 (segment (start 85.5335 58.8198) (end 82.7588 58.8198) (width 0.5) (layer B.Cu) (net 17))
 (segment (start 82.7588 58.8198) (end 81.5335 57.5945) (width 0.5) (layer B.Cu) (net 17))
 (segment (start 96.4553 61.9334) (end 98.1626 61.9334) (width 0.5) (layer B.Cu) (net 17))
 (segment (start 98.1626 61.9334) (end 98.893 62.6638) (width 0.5) (layer B.Cu) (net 17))
 (segment (start 96.393 62.9485) (end 96.393 61.9957) (width 0.5) (layer B.Cu) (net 17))
 (segment (start 96.393 61.9957) (end 96.4553 61.9334) (width 0.5) (layer B.Cu) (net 17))
 (segment (start 98.893 62.6638) (end 99.6234 61.9334) (width 0.5) (layer B.Cu) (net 17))
 (segment (start 99.6234 61.9334) (end 100.6773 61.9334) (width 0.5) (layer B.Cu) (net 17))
 (segment (start 100.6773 61.9334) (end 101.393 62.6491) (width 0.5) (layer B.Cu) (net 17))
 (segment (start 101.393 62.6491) (end 101.393 62.9485) (width 0.5) (layer B.Cu) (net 17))
 (segment (start 98.893 62.9485) (end 98.893 62.6638) (width 0.5) (layer B.Cu) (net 17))
 (segment (start 96.393 64.0715) (end 96.393 62.9485) (width 0.5) (layer B.Cu) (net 17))
 (segment (start 98.893 64.0715) (end 98.893 62.9485) (width 0.5) (layer B.Cu) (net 17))
 (segment (start 101.393 64.0715) (end 101.393 62.9485) (width 0.5) (layer B.Cu) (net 17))
 (segment (start 85.5335 57.5945) (end 85.5335 58.8198) (width 0.5) (layer B.Cu) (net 17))
 (segment (start 81.5335 57.5945) (end 80.295 58.833) (width 0.5) (layer B.Cu) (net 17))
 (segment (start 80.295 58.833) (end 78.772 58.833) (width 0.5) (layer B.Cu) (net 17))
 (segment (start 78.772 58.833) (end 77.5335 57.5945) (width 0.5) (layer B.Cu) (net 17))
 (segment (start 101.393 64.0715) (end 101.393 62.9485) (width 0.5) (layer F.Cu) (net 17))
 (segment (start 98.893 64.0715) (end 98.893 62.9485) (width 0.5) (layer F.Cu) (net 17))
 (segment (start 96.393 64.0715) (end 96.393 62.9485) (width 0.5) (layer F.Cu) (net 17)))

